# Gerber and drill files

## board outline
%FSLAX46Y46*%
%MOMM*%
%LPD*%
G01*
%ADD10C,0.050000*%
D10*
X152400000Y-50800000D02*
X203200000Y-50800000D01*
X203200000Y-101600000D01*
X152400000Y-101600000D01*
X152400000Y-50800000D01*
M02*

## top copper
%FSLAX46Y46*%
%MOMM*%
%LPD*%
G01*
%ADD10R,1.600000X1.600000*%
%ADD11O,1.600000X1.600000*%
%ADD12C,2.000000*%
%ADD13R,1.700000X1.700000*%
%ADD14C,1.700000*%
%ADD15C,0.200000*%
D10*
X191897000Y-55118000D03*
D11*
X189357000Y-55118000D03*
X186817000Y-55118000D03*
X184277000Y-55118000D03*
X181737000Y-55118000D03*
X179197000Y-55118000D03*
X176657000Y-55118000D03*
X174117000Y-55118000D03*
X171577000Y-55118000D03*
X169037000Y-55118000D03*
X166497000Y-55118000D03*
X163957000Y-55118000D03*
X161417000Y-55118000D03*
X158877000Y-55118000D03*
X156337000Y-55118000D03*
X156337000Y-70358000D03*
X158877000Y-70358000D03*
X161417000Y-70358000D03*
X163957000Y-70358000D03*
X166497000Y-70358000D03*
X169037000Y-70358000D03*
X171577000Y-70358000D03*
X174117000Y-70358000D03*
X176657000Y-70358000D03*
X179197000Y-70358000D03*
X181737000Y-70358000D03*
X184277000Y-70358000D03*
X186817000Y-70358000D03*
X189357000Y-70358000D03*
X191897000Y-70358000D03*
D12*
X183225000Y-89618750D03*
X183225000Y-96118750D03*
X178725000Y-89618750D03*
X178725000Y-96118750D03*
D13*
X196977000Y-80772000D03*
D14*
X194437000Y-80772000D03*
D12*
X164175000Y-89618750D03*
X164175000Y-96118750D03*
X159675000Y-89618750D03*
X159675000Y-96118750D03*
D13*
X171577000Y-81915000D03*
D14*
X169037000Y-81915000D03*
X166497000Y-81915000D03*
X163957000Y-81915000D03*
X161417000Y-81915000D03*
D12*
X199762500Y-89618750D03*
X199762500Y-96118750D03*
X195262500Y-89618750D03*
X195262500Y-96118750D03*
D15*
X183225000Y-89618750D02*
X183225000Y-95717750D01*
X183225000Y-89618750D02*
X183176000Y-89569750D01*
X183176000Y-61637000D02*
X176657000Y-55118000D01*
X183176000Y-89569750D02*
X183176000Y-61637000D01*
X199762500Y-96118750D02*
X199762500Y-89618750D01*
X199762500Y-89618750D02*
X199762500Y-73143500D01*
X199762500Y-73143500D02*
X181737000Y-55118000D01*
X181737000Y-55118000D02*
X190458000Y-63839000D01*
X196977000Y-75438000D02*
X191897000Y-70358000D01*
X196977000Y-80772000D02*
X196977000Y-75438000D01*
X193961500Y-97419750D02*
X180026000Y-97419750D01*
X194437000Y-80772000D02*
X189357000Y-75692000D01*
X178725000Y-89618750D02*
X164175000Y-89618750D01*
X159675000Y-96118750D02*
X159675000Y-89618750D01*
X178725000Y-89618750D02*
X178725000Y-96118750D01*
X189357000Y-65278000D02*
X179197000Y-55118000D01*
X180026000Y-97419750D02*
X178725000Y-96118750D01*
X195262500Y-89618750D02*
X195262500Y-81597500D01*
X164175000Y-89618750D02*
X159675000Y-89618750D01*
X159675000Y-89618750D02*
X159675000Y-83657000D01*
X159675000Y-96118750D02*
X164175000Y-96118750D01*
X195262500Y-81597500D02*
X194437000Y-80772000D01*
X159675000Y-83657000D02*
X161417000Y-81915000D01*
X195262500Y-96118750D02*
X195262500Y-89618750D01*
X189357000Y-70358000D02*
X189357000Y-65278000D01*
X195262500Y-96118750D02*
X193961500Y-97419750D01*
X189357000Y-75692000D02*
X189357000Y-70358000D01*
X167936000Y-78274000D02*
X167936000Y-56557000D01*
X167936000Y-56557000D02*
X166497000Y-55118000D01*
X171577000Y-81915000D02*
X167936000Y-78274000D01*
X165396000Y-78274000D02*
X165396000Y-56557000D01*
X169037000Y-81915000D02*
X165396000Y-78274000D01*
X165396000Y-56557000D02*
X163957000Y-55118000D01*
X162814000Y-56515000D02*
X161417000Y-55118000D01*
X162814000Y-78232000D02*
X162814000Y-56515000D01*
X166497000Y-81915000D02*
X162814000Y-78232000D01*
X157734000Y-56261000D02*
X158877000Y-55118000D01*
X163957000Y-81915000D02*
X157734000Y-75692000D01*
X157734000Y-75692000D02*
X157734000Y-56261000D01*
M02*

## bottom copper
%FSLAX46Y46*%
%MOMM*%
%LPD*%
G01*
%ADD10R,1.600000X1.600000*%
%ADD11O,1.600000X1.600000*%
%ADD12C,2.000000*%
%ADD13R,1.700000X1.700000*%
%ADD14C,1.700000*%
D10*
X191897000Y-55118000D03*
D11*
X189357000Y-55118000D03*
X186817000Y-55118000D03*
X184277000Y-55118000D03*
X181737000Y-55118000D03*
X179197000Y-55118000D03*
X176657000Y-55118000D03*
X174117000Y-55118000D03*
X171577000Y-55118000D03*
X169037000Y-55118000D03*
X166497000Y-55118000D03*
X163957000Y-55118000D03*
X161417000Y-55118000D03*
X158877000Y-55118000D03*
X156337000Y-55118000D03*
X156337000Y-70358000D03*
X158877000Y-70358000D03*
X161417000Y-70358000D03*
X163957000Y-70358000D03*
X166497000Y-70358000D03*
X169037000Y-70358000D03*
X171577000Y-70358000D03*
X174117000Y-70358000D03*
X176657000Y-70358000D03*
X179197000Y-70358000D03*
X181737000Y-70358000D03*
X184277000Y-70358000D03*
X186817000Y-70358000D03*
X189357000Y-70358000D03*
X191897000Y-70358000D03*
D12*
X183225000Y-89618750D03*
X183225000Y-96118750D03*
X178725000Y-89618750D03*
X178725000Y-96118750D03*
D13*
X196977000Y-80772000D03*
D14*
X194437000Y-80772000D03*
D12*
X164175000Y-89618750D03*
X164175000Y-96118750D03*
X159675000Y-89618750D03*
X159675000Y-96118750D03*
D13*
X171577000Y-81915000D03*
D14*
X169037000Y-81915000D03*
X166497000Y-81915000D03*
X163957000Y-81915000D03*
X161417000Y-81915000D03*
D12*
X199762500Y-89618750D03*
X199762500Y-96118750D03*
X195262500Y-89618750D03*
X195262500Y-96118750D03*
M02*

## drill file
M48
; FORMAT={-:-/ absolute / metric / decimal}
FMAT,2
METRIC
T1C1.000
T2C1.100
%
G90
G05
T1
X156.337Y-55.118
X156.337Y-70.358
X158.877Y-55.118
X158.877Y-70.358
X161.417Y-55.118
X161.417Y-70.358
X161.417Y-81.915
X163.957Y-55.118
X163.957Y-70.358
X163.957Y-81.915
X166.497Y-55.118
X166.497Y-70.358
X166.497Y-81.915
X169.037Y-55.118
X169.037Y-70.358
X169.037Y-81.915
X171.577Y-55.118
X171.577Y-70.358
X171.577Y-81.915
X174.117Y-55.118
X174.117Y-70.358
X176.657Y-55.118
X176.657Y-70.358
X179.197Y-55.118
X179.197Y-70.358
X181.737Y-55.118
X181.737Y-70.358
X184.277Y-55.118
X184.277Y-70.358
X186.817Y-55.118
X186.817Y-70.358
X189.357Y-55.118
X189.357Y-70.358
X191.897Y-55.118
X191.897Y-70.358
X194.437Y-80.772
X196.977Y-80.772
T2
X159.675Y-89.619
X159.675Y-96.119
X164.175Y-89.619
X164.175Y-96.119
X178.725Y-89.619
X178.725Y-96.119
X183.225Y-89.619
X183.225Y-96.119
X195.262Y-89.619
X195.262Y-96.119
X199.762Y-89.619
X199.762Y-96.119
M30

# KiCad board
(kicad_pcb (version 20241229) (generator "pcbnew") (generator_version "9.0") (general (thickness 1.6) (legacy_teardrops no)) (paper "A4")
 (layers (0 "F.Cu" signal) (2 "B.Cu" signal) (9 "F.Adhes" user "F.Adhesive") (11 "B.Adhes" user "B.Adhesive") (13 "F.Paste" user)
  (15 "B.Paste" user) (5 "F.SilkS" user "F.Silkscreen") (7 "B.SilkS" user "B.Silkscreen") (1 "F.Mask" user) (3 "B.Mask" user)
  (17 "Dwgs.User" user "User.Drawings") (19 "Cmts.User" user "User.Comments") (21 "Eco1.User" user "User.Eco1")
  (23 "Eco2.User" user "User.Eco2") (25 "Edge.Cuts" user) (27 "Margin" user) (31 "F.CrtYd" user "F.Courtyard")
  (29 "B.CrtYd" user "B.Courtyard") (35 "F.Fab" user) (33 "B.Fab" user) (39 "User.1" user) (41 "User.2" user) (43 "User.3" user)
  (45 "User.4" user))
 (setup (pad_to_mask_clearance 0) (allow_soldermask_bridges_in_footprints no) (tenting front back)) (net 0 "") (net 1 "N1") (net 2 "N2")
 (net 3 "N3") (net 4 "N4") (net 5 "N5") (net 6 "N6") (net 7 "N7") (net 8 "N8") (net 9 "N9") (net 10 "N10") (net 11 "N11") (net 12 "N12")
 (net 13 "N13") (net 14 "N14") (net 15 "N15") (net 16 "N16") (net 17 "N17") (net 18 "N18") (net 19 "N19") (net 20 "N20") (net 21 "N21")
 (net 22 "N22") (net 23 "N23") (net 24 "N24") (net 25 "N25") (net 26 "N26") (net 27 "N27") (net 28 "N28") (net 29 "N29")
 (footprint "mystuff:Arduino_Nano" (layer "F.Cu") (at 191.897 55.118 -90)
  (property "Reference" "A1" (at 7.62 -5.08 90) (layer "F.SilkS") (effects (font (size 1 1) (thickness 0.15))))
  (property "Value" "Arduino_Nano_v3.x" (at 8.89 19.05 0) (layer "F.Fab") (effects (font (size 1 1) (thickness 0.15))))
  (pad "1" thru_hole rect (at 0 0 270) (size 1.6 1.6) (drill 1) (layers "*.Cu" "*.Mask") (remove_unused_layers no) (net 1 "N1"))
  (pad "2" thru_hole oval (at 0 2.54 270) (size 1.6 1.6) (drill 1) (layers "*.Cu" "*.Mask") (remove_unused_layers no) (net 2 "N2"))
  (pad "3" thru_hole oval (at 0 5.08 270) (size 1.6 1.6) (drill 1) (layers "*.Cu" "*.Mask") (remove_unused_layers no) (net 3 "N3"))
  (pad "4" thru_hole oval (at 0 7.62 270) (size 1.6 1.6) (drill 1) (layers "*.Cu" "*.Mask") (remove_unused_layers no) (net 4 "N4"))
  (pad "5" thru_hole oval (at 0 10.16 270) (size 1.6 1.6) (drill 1) (layers "*.Cu" "*.Mask") (remove_unused_layers no) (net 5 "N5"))
  (pad "6" thru_hole oval (at 0 12.7 270) (size 1.6 1.6) (drill 1) (layers "*.Cu" "*.Mask") (remove_unused_layers no) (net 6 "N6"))
  (pad "7" thru_hole oval (at 0 15.24 270) (size 1.6 1.6) (drill 1) (layers "*.Cu" "*.Mask") (remove_unused_layers no) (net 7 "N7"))
  (pad "8" thru_hole oval (at 0 17.78 270) (size 1.6 1.6) (drill 1) (layers "*.Cu" "*.Mask") (remove_unused_layers no) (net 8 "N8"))
  (pad "9" thru_hole oval (at 0 20.32 270) (size 1.6 1.6) (drill 1) (layers "*.Cu" "*.Mask") (remove_unused_layers no) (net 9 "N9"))
  (pad "10" thru_hole oval (at 0 22.86 270) (size 1.6 1.6) (drill 1) (layers "*.Cu" "*.Mask") (remove_unused_layers no) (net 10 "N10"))
  (pad "11" thru_hole oval (at 0 25.4 270) (size 1.6 1.6) (drill 1) (layers "*.Cu" "*.Mask") (remove_unused_layers no) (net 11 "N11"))
  (pad "12" thru_hole oval (at 0 27.94 270) (size 1.6 1.6) (drill 1) (layers "*.Cu" "*.Mask") (remove_unused_layers no) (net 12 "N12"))
  (pad "13" thru_hole oval (at 0 30.48 270) (size 1.6 1.6) (drill 1) (layers "*.Cu" "*.Mask") (remove_unused_layers no) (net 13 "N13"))
  (pad "14" thru_hole oval (at 0 33.02 270) (size 1.6 1.6) (drill 1) (layers "*.Cu" "*.Mask") (remove_unused_layers no) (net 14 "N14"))
  (pad "15" thru_hole oval (at 0 35.56 270) (size 1.6 1.6) (drill 1) (layers "*.Cu" "*.Mask") (remove_unused_layers no) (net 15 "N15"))
  (pad "16" thru_hole oval (at 15.24 35.56 270) (size 1.6 1.6) (drill 1) (layers "*.Cu" "*.Mask") (remove_unused_layers no) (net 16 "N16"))
  (pad "17" thru_hole oval (at 15.24 33.02 270) (size 1.6 1.6) (drill 1) (layers "*.Cu" "*.Mask") (remove_unused_layers no) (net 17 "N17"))
  (pad "18" thru_hole oval (at 15.24 30.48 270) (size 1.6 1.6) (drill 1) (layers "*.Cu" "*.Mask") (remove_unused_layers no) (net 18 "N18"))
  (pad "19" thru_hole oval (at 15.24 27.94 270) (size 1.6 1.6) (drill 1) (layers "*.Cu" "*.Mask") (remove_unused_layers no) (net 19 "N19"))
  (pad "20" thru_hole oval (at 15.24 25.4 270) (size 1.6 1.6) (drill 1) (layers "*.Cu" "*.Mask") (remove_unused_layers no) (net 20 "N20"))
  (pad "21" thru_hole oval (at 15.24 22.86 270) (size 1.6 1.6) (drill 1) (layers "*.Cu" "*.Mask") (remove_unused_layers no) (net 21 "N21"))
  (pad "22" thru_hole oval (at 15.24 20.32 270) (size 1.6 1.6) (drill 1) (layers "*.Cu" "*.Mask") (remove_unused_layers no) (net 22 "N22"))
  (pad "23" thru_hole oval (at 15.24 17.78 270) (size 1.6 1.6) (drill 1) (layers "*.Cu" "*.Mask") (remove_unused_layers no) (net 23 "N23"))
  (pad "24" thru_hole oval (at 15.24 15.24 270) (size 1.6 1.6) (drill 1) (layers "*.Cu" "*.Mask") (remove_unused_layers no) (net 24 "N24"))
  (pad "25" thru_hole oval (at 15.24 12.7 270) (size 1.6 1.6) (drill 1) (layers "*.Cu" "*.Mask") (remove_unused_layers no) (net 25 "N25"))
  (pad "26" thru_hole oval (at 15.24 10.16 270) (size 1.6 1.6) (drill 1) (layers "*.Cu" "*.Mask") (remove_unused_layers no) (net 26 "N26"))
  (pad "27" thru_hole oval (at 15.24 7.62 270) (size 1.6 1.6) (drill 1) (layers "*.Cu" "*.Mask") (remove_unused_layers no) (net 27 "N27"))
  (pad "28" thru_hole oval (at 15.24 5.08 270) (size 1.6 1.6) (drill 1) (layers "*.Cu" "*.Mask") (remove_unused_layers no) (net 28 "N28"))
  (pad "29" thru_hole oval (at 15.24 2.54 270) (size 1.6 1.6) (drill 1) (layers "*.Cu" "*.Mask") (remove_unused_layers no) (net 6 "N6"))
  (pad "30" thru_hole oval (at 15.24 0 270) (size 1.6 1.6) (drill 1) (layers "*.Cu" "*.Mask") (remove_unused_layers no) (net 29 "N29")))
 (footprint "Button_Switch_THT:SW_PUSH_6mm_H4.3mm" (layer "F.Cu") (at 183.225 89.61875 -90)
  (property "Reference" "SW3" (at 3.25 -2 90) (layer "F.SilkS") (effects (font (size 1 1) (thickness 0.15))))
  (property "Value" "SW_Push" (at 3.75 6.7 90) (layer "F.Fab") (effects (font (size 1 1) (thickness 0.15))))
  (pad "1" thru_hole circle (at 0 0) (size 2 2) (drill 1.1) (layers "*.Cu" "*.Mask") (remove_unused_layers no) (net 7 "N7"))
  (pad "1" thru_hole circle (at 6.5 0) (size 2 2) (drill 1.1) (layers "*.Cu" "*.Mask") (remove_unused_layers no) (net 7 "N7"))
  (pad "2" thru_hole circle (at 0 4.5) (size 2 2) (drill 1.1) (layers "*.Cu" "*.Mask") (remove_unused_layers no) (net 6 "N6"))
  (pad "2" thru_hole circle (at 6.5 4.5) (size 2 2) (drill 1.1) (layers "*.Cu" "*.Mask") (remove_unused_layers no) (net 6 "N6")))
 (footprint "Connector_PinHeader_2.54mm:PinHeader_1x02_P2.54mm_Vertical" (layer "F.Cu") (at 196.977 80.772 -90)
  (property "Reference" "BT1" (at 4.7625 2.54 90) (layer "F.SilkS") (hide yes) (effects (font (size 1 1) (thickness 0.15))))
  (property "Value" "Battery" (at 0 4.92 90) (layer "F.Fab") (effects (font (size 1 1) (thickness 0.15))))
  (pad "1" thru_hole rect (at 0 0 270) (size 1.7 1.7) (drill 1) (layers "*.Cu" "*.Mask") (remove_unused_layers no) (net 29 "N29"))
  (pad "2" thru_hole circle (at 0 2.54 270) (size 1.7 1.7) (drill 1) (layers "*.Cu" "*.Mask") (remove_unused_layers no) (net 6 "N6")))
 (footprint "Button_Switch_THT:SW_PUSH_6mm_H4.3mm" (layer "F.Cu") (at 164.175 89.61875 -90)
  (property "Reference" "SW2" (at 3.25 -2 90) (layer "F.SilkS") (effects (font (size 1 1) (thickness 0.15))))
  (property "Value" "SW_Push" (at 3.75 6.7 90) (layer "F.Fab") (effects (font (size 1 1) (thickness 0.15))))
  (pad "1" thru_hole circle (at 0 0) (size 2 2) (drill 1.1) (layers "*.Cu" "*.Mask") (remove_unused_layers no) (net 6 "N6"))
  (pad "1" thru_hole circle (at 6.5 0) (size 2 2) (drill 1.1) (layers "*.Cu" "*.Mask") (remove_unused_layers no) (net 6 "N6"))
  (pad "2" thru_hole circle (at 0 4.5) (size 2 2) (drill 1.1) (layers "*.Cu" "*.Mask") (remove_unused_layers no) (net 6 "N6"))
  (pad "2" thru_hole circle (at 6.5 4.5) (size 2 2) (drill 1.1) (layers "*.Cu" "*.Mask") (remove_unused_layers no) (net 6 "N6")))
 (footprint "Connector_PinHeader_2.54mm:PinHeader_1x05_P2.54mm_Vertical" (layer "F.Cu") (at 171.577 81.915 -90)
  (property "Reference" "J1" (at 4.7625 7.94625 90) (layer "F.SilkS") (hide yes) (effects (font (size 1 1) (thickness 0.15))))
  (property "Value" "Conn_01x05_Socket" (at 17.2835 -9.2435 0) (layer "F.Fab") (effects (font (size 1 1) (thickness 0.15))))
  (pad "1" thru_hole rect (at 0 0 270) (size 1.7 1.7) (drill 1) (layers "*.Cu" "*.Mask") (remove_unused_layers no) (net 11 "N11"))
  (pad "2" thru_hole circle (at 0 2.54 270) (size 1.7 1.7) (drill 1) (layers "*.Cu" "*.Mask") (remove_unused_layers no) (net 12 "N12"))
  (pad "3" thru_hole circle (at 0 5.08 270) (size 1.7 1.7) (drill 1) (layers "*.Cu" "*.Mask") (remove_unused_layers no) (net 13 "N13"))
  (pad "4" thru_hole circle (at 0 7.62 270) (size 1.7 1.7) (drill 1) (layers "*.Cu" "*.Mask") (remove_unused_layers no) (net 14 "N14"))
  (pad "5" thru_hole circle (at 0 10.16 270) (size 1.7 1.7) (drill 1) (layers "*.Cu" "*.Mask") (remove_unused_layers no) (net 6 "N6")))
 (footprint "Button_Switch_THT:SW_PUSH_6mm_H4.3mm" (layer "F.Cu") (at 199.7625 89.61875 -90)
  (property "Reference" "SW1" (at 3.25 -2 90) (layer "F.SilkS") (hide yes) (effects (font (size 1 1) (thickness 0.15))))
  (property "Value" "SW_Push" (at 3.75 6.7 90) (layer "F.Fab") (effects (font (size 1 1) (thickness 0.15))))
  (pad "1" thru_hole circle (at 0 0) (size 2 2) (drill 1.1) (layers "*.Cu" "*.Mask") (remove_unused_layers no) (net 5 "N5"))
  (pad "1" thru_hole circle (at 6.5 0) (size 2 2) (drill 1.1) (layers "*.Cu" "*.Mask") (remove_unused_layers no) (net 5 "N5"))
  (pad "2" thru_hole circle (at 0 4.5) (size 2 2) (drill 1.1) (layers "*.Cu" "*.Mask") (remove_unused_layers no) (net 6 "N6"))
  (pad "2" thru_hole circle (at 6.5 4.5) (size 2 2) (drill 1.1) (layers "*.Cu" "*.Mask") (remove_unused_layers no) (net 6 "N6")))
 (gr_rect (start 152.4 50.8) (end 203.2 101.6) (stroke (width 0.05) (type solid)) (fill no) (layer "Edge.Cuts"))
 (segment (start 183.225 89.61875) (end 183.225 95.71775) (width 0.2) (layer "F.Cu") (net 7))
 (segment (start 183.225 89.61875) (end 183.176 89.56975) (width 0.2) (layer "F.Cu") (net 7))
 (segment (start 183.176 61.637) (end 176.657 55.118) (width 0.2) (layer "F.Cu") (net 7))
 (segment (start 183.176 89.56975) (end 183.176 61.637) (width 0.2) (layer "F.Cu") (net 7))
 (segment (start 199.7625 96.11875) (end 199.7625 89.61875) (width 0.2) (layer "F.Cu") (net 5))
 (segment (start 199.7625 89.61875) (end 199.7625 73.1435) (width 0.2) (layer "F.Cu") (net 5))
 (segment (start 199.7625 73.1435) (end 181.737 55.118) (width 0.2) (layer "F.Cu") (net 5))
 (segment (start 181.737 55.118) (end 190.458 63.839) (width 0.2) (layer "F.Cu") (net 5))
 (segment (start 196.977 75.438) (end 191.897 70.358) (width 0.2) (layer "F.Cu") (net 29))
 (segment (start 196.977 80.772) (end 196.977 75.438) (width 0.2) (layer "F.Cu") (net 29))
 (segment (start 193.9615 97.41975) (end 180.026 97.41975) (width 0.2) (layer "F.Cu") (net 6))
 (segment (start 194.437 80.772) (end 189.357 75.692) (width 0.2) (layer "F.Cu") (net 6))
 (segment (start 178.725 89.61875) (end 164.175 89.61875) (width 0.2) (layer "F.Cu") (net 6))
 (segment (start 159.675 96.11875) (end 159.675 89.61875) (width 0.2) (layer "F.Cu") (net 6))
 (segment (start 178.725 89.61875) (end 178.725 96.11875) (width 0.2) (layer "F.Cu") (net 6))
 (segment (start 189.357 65.278) (end 179.197 55.118) (width 0.2) (layer "F.Cu") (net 6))
 (segment (start 180.026 97.41975) (end 178.725 96.11875) (width 0.2) (layer "F.Cu") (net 6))
 (segment (start 195.2625 89.61875) (end 195.2625 81.5975) (width 0.2) (layer "F.Cu") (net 6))
 (segment (start 164.175 89.61875) (end 159.675 89.61875) (width 0.2) (layer "F.Cu") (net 6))
 (segment (start 159.675 89.61875) (end 159.675 83.657) (width 0.2) (layer "F.Cu") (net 6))
 (segment (start 159.675 96.11875) (end 164.175 96.11875) (width 0.2) (layer "F.Cu") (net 6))
 (segment (start 195.2625 81.5975) (end 194.437 80.772) (width 0.2) (layer "F.Cu") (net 6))
 (segment (start 159.675 83.657) (end 161.417 81.915) (width 0.2) (layer "F.Cu") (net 6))
 (segment (start 195.2625 96.11875) (end 195.2625 89.61875) (width 0.2) (layer "F.Cu") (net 6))
 (segment (start 189.357 70.358) (end 189.357 65.278) (width 0.2) (layer "F.Cu") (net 6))
 (segment (start 195.2625 96.11875) (end 193.9615 97.41975) (width 0.2) (layer "F.Cu") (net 6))
 (segment (start 189.357 75.692) (end 189.357 70.358) (width 0.2) (layer "F.Cu") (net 6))
 (segment (start 167.936 78.274) (end 167.936 56.557) (width 0.2) (layer "F.Cu") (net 11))
 (segment (start 167.936 56.557) (end 166.497 55.118) (width 0.2) (layer "F.Cu") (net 11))
 (segment (start 171.577 81.915) (end 167.936 78.274) (width 0.2) (layer "F.Cu") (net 11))
 (segment (start 165.396 78.274) (end 165.396 56.557) (width 0.2) (layer "F.Cu") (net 12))
 (segment (start 169.037 81.915) (end 165.396 78.274) (width 0.2) (layer "F.Cu") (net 12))
 (segment (start 165.396 56.557) (end 163.957 55.118) (width 0.2) (layer "F.Cu") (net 12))
 (segment (start 162.814 56.515) (end 161.417 55.118) (width 0.2) (layer "F.Cu") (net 13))
 (segment (start 162.814 78.232) (end 162.814 56.515) (width 0.2) (layer "F.Cu") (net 13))
 (segment (start 166.497 81.915) (end 162.814 78.232) (width 0.2) (layer "F.Cu") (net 13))
 (segment (start 157.734 56.261) (end 158.877 55.118) (width 0.2) (layer "F.Cu") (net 14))
 (segment (start 163.957 81.915) (end 157.734 75.692) (width 0.2) (layer "F.Cu") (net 14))
 (segment (start 157.734 75.692) (end 157.734 56.261) (width 0.2) (layer "F.Cu") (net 14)))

